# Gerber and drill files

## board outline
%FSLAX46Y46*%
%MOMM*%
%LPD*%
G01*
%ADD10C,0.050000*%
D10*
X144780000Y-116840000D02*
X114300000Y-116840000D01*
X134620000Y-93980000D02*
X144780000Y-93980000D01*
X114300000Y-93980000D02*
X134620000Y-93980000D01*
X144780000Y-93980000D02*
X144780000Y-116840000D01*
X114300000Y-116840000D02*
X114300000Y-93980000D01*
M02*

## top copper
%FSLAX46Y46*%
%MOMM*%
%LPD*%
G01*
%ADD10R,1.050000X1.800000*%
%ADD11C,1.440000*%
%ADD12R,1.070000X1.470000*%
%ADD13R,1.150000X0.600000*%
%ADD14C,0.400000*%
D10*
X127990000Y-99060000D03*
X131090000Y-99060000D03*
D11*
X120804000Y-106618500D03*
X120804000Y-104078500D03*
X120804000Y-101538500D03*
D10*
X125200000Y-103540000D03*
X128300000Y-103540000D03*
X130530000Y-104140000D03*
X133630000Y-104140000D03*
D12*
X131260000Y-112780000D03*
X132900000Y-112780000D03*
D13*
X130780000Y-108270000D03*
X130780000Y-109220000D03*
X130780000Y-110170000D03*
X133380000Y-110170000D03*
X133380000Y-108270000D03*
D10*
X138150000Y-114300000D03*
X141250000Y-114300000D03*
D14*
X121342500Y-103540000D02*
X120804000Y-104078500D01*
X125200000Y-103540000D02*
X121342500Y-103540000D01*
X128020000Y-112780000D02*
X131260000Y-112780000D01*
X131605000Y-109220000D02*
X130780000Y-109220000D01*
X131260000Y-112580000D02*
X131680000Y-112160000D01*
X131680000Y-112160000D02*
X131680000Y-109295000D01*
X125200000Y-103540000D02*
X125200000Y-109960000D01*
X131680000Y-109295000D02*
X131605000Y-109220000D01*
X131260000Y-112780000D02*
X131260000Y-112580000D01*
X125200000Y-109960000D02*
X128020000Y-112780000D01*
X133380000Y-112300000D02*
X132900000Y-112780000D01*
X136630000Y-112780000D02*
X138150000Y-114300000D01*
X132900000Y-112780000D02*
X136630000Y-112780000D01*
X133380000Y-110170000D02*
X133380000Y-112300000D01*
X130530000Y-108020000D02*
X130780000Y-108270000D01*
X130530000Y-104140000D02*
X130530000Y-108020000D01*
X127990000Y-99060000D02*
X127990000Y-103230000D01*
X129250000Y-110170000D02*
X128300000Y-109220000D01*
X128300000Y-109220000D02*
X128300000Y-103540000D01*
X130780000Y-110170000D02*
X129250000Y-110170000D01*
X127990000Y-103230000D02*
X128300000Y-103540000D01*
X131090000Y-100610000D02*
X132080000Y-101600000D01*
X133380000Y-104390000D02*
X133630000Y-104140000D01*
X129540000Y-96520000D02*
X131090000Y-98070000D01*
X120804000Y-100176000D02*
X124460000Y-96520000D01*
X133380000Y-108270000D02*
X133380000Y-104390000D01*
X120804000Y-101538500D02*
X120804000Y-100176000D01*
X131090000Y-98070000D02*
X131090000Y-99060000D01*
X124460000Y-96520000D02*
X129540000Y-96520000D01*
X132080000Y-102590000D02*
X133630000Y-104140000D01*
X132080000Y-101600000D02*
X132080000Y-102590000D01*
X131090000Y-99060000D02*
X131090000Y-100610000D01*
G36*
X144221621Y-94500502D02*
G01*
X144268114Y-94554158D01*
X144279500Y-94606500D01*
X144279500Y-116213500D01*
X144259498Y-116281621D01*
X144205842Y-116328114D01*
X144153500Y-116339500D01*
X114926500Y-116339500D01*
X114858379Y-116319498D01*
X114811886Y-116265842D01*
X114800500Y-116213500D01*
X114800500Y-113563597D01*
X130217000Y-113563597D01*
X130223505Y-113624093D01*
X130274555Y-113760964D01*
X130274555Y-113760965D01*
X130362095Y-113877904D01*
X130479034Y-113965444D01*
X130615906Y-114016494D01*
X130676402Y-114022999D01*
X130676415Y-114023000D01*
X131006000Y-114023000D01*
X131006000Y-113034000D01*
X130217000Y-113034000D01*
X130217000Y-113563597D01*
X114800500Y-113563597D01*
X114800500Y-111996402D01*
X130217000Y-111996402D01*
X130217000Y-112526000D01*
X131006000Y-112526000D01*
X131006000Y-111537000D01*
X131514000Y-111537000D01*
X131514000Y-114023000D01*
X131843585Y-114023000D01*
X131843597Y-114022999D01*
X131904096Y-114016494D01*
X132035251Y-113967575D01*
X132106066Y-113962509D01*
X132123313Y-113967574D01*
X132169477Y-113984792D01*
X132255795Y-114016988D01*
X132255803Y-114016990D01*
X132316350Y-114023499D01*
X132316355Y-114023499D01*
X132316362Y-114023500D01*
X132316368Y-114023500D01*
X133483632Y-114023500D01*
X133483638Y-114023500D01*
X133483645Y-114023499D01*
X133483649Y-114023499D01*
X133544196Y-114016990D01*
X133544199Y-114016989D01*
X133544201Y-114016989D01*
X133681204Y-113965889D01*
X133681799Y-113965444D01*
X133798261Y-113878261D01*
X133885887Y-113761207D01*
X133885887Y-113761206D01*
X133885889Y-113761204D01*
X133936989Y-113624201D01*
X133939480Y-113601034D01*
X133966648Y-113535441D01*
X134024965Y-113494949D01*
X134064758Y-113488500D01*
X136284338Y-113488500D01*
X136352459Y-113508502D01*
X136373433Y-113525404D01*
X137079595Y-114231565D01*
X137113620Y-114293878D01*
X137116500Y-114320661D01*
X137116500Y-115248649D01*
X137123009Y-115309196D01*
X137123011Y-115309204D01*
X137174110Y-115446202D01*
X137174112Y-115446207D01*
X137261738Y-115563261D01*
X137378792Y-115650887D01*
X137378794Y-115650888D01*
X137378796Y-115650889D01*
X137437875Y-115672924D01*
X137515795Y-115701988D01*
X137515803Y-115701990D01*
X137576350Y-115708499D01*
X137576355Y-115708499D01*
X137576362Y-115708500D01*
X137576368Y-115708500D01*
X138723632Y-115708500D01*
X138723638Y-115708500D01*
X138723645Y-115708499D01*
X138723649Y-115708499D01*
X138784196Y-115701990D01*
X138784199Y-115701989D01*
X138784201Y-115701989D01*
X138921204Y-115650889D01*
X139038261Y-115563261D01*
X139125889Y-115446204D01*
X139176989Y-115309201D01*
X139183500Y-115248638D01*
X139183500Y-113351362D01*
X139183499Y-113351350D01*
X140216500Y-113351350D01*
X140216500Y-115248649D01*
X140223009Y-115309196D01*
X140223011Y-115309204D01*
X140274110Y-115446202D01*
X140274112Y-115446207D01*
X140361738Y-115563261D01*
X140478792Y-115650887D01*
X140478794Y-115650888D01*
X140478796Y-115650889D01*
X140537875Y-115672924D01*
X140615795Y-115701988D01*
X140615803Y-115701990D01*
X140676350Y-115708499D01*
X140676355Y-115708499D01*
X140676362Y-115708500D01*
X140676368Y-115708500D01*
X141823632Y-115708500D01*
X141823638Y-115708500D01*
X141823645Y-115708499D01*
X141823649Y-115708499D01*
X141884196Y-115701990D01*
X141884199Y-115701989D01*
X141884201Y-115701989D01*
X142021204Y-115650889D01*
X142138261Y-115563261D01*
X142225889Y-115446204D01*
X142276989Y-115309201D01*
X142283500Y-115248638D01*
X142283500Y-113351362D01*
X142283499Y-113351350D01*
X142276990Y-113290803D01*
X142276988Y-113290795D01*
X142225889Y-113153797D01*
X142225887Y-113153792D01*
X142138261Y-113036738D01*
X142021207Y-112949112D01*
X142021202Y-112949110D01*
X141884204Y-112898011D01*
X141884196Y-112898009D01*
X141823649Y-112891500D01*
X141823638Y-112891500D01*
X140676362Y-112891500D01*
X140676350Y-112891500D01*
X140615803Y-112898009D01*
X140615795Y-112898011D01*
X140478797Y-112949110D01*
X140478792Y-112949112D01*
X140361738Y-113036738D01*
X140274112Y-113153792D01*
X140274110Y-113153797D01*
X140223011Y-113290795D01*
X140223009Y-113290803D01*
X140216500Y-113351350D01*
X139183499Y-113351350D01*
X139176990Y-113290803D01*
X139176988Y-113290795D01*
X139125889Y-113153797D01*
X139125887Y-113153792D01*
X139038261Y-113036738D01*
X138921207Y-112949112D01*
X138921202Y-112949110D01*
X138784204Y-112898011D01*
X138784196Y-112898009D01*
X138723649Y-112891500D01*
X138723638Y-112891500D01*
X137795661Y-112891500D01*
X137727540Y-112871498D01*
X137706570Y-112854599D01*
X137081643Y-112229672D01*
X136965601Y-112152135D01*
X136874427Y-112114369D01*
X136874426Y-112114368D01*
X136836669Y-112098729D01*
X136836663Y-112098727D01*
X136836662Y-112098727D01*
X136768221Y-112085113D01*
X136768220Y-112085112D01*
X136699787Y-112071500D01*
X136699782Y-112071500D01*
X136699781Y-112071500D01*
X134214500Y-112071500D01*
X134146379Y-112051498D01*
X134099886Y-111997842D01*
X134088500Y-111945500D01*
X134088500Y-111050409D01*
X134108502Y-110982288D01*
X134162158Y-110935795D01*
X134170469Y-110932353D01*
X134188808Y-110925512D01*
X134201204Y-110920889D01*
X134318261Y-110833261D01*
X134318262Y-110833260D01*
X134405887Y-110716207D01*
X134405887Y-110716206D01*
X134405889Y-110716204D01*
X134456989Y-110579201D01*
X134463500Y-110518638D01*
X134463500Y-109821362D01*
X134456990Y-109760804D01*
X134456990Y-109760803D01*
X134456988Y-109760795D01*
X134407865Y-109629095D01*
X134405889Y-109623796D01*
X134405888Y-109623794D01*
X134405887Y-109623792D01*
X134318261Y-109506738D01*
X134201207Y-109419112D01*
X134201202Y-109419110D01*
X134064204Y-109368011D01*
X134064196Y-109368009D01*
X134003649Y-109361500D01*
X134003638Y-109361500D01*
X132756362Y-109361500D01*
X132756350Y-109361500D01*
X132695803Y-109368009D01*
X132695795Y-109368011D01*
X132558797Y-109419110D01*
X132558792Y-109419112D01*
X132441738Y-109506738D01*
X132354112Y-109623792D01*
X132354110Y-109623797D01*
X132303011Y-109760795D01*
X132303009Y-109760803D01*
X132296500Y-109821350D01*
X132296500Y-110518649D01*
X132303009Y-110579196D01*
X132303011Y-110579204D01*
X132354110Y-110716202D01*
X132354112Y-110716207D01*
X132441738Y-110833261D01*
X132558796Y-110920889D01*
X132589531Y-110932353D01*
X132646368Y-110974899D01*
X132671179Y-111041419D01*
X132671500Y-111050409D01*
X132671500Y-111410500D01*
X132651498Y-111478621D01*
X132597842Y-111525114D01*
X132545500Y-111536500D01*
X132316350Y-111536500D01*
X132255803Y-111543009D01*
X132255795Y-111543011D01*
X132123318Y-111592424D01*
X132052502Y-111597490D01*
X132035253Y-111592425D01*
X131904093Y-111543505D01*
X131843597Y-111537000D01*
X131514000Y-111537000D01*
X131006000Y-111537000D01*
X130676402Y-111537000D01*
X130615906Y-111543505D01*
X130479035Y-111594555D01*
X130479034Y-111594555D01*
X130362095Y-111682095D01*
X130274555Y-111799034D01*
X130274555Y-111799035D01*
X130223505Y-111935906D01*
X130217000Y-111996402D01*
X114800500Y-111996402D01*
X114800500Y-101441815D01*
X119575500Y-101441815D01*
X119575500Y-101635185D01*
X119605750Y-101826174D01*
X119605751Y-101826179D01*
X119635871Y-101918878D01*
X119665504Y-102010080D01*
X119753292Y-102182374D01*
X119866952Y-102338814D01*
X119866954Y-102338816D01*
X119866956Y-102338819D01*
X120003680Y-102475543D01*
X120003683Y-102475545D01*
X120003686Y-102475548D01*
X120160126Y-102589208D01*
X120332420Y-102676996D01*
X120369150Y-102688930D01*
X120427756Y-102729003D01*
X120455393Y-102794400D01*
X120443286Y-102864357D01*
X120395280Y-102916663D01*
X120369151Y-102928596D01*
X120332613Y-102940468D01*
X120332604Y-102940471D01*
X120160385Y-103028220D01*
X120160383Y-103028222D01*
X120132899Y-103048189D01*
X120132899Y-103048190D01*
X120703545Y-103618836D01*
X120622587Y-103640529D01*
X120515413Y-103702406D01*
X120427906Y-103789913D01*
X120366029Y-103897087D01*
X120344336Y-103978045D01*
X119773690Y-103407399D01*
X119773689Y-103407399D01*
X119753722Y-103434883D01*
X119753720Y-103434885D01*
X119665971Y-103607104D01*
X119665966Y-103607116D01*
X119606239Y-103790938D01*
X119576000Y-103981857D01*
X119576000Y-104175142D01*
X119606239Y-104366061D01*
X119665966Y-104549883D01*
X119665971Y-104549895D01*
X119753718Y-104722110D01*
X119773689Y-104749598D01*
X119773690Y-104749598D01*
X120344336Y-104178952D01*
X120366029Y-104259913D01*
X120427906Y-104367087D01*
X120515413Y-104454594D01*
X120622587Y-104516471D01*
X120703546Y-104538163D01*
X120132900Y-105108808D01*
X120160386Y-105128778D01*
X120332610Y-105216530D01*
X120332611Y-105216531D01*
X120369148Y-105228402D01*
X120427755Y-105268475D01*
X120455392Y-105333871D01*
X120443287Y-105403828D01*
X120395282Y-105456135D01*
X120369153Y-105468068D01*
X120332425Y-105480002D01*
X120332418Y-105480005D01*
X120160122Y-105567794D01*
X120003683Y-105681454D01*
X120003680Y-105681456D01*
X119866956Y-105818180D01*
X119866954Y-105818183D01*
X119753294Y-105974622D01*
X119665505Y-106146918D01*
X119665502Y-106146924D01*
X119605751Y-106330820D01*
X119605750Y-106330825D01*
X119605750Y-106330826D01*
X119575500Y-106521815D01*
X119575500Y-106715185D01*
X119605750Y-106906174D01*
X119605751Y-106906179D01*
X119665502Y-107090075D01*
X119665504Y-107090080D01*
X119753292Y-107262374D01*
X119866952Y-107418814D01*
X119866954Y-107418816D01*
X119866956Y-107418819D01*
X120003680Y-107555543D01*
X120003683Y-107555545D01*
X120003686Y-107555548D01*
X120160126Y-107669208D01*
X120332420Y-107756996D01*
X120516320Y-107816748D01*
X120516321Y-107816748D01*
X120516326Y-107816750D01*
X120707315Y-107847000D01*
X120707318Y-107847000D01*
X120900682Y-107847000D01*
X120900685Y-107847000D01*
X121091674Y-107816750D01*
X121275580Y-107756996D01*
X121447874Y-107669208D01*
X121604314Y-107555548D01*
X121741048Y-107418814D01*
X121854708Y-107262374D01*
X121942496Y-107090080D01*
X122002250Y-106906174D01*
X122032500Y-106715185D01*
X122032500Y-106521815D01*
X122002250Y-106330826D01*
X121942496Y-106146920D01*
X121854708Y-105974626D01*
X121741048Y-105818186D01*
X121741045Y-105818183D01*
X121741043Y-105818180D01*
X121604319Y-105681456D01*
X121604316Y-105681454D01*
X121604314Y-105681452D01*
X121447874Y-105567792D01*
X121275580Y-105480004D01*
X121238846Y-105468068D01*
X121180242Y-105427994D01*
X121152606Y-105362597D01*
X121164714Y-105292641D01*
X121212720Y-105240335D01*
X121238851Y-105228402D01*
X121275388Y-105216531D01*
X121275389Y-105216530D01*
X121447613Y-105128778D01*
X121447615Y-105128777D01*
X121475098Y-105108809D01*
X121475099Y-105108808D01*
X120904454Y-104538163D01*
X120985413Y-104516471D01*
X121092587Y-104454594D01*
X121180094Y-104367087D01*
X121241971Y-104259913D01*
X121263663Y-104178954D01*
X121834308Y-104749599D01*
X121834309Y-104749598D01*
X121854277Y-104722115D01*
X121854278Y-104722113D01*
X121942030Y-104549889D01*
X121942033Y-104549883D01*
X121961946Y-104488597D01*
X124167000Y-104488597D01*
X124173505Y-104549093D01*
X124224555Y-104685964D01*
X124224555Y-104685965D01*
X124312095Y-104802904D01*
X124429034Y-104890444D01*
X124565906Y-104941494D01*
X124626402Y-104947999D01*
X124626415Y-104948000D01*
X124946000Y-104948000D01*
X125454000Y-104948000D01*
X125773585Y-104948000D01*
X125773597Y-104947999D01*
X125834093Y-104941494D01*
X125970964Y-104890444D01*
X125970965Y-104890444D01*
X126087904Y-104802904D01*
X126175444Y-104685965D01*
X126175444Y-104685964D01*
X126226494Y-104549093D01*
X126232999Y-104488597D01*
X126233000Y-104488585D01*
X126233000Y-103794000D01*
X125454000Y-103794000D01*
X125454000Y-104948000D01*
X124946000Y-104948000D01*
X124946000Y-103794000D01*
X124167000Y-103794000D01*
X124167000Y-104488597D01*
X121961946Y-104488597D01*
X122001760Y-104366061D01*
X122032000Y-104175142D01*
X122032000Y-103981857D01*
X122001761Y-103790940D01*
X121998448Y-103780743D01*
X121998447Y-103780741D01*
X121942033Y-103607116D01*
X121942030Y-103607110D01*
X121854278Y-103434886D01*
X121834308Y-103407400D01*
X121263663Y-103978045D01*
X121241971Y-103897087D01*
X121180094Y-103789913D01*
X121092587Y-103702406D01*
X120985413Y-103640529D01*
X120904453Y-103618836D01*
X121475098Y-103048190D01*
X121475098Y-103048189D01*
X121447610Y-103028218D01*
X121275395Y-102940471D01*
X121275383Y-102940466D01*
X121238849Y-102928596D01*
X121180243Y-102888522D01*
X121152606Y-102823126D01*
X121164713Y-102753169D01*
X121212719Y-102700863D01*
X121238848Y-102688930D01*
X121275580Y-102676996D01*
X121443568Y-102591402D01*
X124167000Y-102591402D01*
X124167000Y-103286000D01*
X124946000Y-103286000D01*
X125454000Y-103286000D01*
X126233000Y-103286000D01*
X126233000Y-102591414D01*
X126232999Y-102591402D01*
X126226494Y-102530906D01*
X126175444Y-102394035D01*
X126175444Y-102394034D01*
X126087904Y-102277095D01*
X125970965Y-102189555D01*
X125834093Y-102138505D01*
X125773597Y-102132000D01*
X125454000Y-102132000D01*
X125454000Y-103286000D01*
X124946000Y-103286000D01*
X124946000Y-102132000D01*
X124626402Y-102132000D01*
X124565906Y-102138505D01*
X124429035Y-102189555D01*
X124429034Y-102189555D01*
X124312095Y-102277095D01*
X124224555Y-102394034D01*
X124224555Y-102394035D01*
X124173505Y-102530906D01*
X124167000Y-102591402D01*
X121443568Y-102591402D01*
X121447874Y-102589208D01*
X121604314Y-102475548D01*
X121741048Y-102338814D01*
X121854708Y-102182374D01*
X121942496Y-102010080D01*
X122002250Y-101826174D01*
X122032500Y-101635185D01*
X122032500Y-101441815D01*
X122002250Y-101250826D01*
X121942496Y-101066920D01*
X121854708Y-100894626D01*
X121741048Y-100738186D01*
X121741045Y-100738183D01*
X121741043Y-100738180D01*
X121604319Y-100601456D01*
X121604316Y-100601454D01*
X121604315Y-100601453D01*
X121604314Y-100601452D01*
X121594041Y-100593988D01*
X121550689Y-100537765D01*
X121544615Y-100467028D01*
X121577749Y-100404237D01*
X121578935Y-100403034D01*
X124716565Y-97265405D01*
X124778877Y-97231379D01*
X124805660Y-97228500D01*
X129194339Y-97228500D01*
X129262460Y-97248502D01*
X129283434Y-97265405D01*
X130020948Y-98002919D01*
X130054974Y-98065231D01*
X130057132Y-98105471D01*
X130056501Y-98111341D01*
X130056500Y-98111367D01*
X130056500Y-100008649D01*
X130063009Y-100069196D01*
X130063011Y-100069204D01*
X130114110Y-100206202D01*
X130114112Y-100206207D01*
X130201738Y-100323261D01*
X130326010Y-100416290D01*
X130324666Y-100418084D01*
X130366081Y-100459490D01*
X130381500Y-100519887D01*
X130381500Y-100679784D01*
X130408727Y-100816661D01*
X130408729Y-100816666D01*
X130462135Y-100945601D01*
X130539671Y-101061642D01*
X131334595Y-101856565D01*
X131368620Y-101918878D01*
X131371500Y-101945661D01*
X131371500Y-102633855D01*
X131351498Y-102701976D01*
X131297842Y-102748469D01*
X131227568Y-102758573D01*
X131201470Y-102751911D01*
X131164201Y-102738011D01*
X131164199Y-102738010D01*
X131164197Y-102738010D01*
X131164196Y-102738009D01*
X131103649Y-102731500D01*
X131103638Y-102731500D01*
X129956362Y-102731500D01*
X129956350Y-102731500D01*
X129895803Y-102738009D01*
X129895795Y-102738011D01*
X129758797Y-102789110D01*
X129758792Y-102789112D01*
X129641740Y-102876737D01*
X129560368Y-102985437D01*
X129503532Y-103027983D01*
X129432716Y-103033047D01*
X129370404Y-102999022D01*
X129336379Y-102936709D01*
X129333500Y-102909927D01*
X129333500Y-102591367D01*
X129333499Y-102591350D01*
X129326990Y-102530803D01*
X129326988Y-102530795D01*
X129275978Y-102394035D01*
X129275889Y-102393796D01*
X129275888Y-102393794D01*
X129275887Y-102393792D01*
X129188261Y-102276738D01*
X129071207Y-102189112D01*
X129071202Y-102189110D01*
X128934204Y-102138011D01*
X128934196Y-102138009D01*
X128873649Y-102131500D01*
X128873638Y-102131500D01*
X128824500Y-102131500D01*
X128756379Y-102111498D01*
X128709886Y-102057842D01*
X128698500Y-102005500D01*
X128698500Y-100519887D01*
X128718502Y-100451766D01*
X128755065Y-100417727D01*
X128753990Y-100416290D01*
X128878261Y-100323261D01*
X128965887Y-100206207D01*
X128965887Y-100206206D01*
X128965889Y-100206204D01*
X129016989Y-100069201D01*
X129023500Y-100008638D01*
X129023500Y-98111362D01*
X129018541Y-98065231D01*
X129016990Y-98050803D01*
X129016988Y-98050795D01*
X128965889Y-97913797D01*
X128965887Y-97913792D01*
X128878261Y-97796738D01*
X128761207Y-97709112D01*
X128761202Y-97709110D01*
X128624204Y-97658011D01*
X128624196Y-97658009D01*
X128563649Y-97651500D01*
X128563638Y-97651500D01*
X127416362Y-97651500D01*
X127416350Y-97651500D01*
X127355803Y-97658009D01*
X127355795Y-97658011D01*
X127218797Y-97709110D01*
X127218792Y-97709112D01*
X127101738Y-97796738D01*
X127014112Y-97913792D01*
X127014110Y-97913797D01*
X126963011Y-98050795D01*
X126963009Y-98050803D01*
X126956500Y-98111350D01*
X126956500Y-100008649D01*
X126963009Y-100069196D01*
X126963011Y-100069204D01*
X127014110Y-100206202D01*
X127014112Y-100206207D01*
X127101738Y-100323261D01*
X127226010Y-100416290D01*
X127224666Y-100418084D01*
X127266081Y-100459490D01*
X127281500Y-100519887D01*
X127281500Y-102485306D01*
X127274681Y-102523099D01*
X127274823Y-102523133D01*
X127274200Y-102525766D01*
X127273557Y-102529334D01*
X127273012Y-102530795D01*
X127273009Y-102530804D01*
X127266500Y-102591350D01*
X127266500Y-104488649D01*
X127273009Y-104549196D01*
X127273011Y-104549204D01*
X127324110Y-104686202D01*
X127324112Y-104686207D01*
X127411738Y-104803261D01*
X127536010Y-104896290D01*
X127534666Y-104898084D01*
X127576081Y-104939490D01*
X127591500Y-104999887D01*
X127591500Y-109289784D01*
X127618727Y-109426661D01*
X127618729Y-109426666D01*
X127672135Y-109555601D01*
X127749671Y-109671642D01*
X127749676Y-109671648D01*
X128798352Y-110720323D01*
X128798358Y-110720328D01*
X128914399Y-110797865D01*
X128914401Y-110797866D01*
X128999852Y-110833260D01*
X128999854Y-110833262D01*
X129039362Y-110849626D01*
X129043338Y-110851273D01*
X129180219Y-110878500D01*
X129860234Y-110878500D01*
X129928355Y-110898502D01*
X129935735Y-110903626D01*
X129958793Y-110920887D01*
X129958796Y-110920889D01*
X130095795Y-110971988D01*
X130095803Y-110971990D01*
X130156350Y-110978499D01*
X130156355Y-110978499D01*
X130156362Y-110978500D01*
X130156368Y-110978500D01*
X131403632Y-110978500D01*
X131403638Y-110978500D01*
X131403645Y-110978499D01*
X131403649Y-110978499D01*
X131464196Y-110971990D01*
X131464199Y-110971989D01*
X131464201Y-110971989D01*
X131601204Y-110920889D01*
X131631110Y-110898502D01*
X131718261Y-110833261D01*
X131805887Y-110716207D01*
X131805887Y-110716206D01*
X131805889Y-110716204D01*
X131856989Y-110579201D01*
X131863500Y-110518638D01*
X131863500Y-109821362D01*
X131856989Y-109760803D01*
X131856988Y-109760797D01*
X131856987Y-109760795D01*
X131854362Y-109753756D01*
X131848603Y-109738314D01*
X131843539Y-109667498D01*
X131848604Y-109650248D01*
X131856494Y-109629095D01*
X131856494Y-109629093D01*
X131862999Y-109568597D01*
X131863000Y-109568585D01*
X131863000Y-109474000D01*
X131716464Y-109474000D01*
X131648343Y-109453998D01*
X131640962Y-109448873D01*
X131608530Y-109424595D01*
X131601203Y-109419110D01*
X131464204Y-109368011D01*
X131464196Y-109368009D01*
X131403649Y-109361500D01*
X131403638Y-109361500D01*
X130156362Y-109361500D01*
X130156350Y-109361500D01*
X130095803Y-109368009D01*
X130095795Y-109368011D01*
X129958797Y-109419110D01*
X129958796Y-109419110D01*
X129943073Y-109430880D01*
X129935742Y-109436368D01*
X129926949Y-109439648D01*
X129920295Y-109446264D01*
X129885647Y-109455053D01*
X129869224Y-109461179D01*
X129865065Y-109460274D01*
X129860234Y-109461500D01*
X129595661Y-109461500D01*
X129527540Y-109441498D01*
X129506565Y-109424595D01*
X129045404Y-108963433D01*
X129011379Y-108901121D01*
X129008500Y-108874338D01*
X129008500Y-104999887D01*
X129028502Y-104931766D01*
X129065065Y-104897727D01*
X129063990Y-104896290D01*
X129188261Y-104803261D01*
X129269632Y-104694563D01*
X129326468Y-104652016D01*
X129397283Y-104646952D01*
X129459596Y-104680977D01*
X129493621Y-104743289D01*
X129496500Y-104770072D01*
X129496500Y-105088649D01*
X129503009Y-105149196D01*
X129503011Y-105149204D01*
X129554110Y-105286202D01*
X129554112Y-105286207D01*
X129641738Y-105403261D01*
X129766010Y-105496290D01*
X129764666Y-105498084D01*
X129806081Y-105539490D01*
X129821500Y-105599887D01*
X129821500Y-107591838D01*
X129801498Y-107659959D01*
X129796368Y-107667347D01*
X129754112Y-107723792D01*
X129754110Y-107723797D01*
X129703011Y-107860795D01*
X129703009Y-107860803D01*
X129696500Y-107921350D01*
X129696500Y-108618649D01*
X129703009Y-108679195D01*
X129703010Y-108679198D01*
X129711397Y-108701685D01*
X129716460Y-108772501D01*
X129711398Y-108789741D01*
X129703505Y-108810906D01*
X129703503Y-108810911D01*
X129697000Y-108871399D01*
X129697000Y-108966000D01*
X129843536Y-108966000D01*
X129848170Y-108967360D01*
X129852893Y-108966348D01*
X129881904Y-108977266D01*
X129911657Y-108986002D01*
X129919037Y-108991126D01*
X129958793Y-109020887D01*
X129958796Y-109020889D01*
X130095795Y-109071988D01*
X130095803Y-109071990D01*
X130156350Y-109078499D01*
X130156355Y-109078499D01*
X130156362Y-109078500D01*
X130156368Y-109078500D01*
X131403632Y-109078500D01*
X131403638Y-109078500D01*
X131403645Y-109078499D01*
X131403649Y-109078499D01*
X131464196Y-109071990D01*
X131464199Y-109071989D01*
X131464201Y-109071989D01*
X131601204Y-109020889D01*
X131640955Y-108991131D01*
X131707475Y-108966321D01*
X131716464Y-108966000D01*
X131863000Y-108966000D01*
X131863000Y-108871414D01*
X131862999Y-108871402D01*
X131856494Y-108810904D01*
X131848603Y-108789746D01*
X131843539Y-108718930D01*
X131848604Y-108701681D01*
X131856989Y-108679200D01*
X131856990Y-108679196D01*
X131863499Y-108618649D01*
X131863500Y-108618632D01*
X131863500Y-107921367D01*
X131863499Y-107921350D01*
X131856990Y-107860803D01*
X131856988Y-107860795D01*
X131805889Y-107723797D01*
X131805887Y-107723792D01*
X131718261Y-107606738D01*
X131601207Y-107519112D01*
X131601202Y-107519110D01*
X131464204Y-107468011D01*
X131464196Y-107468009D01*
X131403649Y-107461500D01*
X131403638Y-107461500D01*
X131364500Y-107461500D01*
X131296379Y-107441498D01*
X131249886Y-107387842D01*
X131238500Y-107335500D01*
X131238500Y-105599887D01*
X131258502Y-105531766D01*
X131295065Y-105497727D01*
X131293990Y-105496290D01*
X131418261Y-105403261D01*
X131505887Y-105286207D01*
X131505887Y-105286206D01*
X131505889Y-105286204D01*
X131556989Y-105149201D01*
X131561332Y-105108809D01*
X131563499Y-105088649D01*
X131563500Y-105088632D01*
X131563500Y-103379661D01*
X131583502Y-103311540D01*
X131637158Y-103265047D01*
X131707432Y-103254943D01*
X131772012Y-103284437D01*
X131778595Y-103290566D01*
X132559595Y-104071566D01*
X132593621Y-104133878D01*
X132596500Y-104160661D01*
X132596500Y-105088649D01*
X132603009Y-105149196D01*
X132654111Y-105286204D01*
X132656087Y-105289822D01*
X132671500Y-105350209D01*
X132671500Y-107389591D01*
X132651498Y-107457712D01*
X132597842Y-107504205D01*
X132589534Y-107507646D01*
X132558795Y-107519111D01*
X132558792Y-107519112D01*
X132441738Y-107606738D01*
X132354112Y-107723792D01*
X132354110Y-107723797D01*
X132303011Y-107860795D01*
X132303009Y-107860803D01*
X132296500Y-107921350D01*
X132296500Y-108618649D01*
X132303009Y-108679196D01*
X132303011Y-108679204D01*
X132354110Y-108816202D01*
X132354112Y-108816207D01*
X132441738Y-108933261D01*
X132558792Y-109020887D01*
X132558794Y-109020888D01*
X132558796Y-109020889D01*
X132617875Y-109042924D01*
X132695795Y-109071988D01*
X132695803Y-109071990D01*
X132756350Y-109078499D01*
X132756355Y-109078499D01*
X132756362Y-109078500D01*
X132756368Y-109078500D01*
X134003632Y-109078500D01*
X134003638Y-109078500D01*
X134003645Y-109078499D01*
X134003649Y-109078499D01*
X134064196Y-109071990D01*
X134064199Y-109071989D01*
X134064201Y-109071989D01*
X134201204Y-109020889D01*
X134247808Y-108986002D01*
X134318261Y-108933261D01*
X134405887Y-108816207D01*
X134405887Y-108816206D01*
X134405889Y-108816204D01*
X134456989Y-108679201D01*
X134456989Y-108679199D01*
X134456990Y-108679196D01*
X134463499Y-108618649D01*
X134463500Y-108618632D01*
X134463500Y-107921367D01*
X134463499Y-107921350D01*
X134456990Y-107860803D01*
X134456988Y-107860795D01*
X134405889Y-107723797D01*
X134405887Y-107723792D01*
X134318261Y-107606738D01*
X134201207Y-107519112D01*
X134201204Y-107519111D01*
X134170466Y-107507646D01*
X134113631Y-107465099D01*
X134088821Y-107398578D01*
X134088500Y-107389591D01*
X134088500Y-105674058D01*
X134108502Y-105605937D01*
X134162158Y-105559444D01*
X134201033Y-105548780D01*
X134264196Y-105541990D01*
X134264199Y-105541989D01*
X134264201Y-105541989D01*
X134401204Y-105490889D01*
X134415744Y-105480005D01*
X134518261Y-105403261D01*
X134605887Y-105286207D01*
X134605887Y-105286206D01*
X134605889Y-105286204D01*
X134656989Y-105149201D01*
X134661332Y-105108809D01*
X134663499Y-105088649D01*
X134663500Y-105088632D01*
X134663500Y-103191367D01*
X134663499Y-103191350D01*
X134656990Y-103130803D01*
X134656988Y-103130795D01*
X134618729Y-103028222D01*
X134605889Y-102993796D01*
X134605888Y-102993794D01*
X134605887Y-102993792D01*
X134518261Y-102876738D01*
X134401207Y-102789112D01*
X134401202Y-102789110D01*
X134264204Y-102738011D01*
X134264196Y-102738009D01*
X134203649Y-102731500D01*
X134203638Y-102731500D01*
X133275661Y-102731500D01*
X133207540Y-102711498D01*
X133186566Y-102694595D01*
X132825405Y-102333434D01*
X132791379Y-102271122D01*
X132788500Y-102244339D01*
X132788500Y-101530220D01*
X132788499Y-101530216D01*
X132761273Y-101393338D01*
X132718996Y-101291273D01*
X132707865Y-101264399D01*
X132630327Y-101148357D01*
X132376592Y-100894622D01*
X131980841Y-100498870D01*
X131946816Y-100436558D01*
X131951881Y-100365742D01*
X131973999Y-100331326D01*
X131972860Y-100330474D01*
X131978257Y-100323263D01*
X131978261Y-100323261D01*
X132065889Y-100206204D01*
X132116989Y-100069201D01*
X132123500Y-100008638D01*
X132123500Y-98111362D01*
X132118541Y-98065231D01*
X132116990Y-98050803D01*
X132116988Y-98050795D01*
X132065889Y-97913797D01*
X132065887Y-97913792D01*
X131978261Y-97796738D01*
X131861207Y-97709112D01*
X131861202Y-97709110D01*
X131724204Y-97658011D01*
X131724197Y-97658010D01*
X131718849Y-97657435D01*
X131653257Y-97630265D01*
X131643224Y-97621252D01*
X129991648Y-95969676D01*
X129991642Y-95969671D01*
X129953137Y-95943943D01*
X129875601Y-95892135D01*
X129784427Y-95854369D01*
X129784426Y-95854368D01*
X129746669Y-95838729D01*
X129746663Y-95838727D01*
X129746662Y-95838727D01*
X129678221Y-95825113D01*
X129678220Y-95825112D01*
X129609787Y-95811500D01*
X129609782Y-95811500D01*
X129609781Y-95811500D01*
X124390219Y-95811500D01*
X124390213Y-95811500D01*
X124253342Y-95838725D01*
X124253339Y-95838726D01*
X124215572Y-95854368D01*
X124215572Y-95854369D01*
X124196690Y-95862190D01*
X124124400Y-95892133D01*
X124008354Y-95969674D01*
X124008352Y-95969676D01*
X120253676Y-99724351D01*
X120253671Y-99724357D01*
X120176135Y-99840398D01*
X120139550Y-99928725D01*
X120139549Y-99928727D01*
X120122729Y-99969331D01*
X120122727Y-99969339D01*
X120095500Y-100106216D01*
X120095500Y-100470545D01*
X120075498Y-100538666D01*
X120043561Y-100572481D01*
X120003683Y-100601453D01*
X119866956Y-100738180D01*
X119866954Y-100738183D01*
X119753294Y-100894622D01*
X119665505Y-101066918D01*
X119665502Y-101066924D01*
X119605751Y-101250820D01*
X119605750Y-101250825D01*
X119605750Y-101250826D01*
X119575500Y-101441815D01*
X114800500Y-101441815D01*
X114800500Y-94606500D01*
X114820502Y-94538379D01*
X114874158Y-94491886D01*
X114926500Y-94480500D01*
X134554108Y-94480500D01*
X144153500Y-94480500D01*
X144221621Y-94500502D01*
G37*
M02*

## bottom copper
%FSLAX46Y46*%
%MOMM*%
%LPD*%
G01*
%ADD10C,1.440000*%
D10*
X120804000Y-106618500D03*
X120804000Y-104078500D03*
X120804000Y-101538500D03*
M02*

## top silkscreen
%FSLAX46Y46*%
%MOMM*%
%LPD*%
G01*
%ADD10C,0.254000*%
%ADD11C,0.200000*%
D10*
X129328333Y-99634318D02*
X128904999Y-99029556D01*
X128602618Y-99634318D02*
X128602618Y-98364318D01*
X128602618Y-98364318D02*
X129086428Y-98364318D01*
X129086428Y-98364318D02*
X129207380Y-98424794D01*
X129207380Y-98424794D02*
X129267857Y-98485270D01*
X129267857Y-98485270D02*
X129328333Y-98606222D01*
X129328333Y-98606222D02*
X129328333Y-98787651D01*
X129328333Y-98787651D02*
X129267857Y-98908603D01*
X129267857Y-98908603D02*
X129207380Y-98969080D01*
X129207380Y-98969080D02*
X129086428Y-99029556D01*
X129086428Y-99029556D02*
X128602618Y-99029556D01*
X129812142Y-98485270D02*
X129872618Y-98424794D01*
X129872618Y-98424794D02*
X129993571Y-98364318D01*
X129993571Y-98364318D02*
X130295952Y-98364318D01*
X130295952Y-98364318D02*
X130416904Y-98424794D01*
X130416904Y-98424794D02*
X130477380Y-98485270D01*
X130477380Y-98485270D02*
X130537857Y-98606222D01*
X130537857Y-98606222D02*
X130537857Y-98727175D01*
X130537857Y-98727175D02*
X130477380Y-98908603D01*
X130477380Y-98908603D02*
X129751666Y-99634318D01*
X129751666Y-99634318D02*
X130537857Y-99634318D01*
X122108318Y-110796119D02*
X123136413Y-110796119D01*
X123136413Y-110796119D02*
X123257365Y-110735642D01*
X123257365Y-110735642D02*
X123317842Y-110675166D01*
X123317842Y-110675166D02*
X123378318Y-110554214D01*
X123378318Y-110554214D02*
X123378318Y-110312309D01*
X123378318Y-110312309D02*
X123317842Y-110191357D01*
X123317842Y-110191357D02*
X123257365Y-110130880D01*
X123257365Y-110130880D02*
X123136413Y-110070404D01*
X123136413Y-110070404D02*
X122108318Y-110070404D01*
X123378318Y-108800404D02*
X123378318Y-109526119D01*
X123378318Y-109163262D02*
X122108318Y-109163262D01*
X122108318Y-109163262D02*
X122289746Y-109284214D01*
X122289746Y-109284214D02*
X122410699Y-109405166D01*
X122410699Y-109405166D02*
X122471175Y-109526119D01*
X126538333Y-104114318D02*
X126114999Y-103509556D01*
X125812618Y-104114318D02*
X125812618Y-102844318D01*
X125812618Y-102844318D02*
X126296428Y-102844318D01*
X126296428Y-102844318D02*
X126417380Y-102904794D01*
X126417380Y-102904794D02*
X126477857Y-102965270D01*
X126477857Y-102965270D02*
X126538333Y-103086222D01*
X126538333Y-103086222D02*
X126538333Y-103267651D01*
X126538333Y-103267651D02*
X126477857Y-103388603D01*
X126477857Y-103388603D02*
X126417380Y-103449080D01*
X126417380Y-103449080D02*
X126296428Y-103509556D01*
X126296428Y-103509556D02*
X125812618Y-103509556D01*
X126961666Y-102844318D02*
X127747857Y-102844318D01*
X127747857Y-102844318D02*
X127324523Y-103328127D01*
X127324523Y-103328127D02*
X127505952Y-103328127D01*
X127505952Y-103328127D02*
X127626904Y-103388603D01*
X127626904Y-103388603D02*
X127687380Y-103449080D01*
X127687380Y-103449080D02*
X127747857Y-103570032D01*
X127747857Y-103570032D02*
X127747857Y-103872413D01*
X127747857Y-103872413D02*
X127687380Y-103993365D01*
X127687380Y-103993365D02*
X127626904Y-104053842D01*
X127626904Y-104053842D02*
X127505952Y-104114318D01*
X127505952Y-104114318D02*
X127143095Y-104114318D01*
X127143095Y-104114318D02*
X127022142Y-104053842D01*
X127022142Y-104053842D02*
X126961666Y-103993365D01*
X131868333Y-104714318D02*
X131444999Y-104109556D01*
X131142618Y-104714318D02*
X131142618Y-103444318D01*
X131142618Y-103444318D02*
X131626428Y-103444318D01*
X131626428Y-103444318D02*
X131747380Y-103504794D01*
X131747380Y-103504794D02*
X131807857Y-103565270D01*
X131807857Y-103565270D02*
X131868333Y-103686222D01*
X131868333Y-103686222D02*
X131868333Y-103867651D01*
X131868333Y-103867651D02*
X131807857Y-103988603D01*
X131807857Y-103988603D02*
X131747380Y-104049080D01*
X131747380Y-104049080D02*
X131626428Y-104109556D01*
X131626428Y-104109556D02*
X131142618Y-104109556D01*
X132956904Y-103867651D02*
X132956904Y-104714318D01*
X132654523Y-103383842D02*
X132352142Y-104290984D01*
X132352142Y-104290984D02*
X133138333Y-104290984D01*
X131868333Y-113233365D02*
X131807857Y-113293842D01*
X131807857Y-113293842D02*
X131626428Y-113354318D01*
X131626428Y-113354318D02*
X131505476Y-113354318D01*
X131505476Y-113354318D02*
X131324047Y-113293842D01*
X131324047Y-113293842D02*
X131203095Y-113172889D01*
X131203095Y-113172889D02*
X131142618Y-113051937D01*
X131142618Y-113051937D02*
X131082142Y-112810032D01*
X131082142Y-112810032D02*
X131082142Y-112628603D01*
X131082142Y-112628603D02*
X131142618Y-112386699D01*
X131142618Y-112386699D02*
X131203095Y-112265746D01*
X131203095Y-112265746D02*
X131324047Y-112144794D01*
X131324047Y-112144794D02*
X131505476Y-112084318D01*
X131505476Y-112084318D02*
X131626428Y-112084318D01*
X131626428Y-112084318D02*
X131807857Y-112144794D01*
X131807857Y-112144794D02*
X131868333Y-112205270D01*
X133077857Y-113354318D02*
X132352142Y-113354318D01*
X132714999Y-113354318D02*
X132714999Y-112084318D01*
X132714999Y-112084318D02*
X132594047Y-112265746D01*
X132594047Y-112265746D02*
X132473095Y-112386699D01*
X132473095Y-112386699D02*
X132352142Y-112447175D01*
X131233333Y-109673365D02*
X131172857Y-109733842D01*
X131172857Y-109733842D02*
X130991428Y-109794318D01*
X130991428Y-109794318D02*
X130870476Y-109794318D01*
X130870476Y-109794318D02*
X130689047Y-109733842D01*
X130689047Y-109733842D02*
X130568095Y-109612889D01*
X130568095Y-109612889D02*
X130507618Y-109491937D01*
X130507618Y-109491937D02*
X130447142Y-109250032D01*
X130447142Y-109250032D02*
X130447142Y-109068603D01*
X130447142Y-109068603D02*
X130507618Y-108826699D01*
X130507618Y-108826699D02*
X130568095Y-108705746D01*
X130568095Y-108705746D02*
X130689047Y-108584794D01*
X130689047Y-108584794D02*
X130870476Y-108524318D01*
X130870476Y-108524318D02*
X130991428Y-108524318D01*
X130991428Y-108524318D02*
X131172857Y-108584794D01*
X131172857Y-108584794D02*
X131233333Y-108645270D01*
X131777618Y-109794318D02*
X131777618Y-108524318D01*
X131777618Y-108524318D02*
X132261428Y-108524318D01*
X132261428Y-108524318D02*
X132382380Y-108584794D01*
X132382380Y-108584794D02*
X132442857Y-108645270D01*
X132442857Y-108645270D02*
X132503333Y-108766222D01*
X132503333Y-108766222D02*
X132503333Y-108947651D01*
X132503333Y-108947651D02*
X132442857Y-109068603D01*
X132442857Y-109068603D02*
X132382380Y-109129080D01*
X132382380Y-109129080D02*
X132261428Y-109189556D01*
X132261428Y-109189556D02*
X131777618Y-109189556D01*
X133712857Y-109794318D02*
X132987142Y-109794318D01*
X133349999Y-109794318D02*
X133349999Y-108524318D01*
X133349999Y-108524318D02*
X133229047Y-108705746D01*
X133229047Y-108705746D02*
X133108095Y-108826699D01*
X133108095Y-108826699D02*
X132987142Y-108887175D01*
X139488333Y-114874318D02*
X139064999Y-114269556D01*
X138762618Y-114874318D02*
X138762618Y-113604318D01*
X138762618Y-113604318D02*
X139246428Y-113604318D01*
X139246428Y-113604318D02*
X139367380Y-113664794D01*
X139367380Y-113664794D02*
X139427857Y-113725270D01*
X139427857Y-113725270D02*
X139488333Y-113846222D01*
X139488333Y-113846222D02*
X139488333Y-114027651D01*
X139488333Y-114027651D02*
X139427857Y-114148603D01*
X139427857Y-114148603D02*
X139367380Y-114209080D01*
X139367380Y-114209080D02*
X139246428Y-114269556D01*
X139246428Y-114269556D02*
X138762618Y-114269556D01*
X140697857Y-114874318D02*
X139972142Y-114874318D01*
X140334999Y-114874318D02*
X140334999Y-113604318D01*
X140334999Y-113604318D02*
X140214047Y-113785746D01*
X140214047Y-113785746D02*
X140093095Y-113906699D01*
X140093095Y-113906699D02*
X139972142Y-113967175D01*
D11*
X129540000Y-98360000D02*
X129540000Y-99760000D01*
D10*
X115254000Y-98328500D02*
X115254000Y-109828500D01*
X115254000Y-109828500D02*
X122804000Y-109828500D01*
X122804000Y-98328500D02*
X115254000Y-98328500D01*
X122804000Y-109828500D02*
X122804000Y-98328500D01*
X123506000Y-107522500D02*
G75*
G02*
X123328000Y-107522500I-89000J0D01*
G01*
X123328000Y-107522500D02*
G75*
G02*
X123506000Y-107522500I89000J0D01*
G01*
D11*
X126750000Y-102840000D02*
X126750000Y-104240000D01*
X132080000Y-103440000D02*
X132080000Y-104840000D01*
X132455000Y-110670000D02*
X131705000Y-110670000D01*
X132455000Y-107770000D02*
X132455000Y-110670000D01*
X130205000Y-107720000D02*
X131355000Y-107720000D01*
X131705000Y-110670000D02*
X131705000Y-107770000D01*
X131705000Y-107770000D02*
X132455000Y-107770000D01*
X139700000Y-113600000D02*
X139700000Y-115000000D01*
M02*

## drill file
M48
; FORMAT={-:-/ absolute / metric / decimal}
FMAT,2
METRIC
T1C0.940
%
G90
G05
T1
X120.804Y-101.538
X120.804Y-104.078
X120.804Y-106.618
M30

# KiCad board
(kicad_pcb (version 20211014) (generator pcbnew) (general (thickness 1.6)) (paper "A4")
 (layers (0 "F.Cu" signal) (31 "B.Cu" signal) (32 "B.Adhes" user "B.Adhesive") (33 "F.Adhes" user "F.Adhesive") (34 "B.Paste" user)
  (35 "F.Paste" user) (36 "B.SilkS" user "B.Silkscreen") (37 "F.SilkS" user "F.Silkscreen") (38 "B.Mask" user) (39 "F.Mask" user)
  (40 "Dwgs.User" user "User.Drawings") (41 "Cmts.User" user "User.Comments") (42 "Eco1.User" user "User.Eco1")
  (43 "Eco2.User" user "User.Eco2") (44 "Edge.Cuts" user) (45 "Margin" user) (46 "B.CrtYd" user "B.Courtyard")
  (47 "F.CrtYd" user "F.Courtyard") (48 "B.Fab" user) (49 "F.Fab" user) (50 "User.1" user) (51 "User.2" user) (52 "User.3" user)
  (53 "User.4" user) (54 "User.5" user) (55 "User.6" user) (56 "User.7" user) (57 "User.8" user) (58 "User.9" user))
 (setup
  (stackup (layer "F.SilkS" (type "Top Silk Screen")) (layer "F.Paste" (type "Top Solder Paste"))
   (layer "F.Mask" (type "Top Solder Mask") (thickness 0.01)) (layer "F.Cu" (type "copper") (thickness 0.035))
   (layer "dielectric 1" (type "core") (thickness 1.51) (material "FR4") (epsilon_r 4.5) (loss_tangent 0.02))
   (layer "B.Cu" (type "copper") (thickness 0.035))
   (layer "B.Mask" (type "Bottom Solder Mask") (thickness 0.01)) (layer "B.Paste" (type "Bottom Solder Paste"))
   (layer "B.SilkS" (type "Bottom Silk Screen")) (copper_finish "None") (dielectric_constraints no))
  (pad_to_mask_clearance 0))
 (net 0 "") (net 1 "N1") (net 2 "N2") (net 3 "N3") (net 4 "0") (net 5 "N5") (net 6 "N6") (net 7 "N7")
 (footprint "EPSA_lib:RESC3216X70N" (layer "F.Cu") (at 129.54 99.06)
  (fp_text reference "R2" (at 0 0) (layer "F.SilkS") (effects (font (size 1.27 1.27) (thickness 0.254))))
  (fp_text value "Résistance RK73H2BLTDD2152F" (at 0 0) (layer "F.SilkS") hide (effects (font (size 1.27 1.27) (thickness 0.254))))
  (fp_line (start 0 -0.7) (end 0 0.7) (layer "F.SilkS") (width 0.2))
  (pad "1" smd rect (at -1.55 0) (size 1.05 1.8) (layers "F.Cu" "F.Paste" "F.Mask") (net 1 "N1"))
  (pad "2" smd rect (at 1.55 0) (size 1.05 1.8) (layers "F.Cu" "F.Paste" "F.Mask") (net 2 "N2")))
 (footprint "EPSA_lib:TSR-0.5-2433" (layer "F.Cu") (at 122.804 109.8285 90)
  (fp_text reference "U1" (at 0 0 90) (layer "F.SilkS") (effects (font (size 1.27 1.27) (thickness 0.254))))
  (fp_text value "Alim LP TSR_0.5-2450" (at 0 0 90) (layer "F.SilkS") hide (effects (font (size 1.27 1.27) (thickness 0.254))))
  (fp_line (start 11.5 -7.55) (end 0 -7.55) (layer "F.SilkS") (width 0.254))
  (fp_line (start 0 -7.55) (end 0 0) (layer "F.SilkS") (width 0.254))
  (fp_line (start 11.5 0) (end 11.5 -7.55) (layer "F.SilkS") (width 0.254))
  (fp_line (start 0 0) (end 11.5 0) (layer "F.SilkS") (width 0.254))
  (fp_circle (center 2.306 0.613) (end 2.306 0.702) (layer "F.SilkS") (width 0.254) (fill none))
  (pad "1" thru_hole circle (at 3.21 -2 90) (size 1.44 1.44) (drill 0.94) (layers *.Cu *.Mask) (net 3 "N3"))
  (pad "2" thru_hole circle (at 5.75 -2 90) (size 1.44 1.44) (drill 0.94) (layers *.Cu *.Mask) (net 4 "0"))
  (pad "3" thru_hole circle (at 8.29 -2 90) (size 1.44 1.44) (drill 0.94) (layers *.Cu *.Mask) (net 2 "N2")))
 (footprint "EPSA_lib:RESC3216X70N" (layer "F.Cu") (at 126.75 103.54)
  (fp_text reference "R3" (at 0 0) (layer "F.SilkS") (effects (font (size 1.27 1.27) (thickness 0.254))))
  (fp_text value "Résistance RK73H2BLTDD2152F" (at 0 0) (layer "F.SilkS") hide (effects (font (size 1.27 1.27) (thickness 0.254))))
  (fp_line (start 0 -0.7) (end 0 0.7) (layer "F.SilkS") (width 0.2))
  (pad "1" smd rect (at -1.55 0) (size 1.05 1.8) (layers "F.Cu" "F.Paste" "F.Mask") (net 4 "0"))
  (pad "2" smd rect (at 1.55 0) (size 1.05 1.8) (layers "F.Cu" "F.Paste" "F.Mask") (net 1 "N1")))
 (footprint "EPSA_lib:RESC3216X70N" (layer "F.Cu") (at 132.08 104.14)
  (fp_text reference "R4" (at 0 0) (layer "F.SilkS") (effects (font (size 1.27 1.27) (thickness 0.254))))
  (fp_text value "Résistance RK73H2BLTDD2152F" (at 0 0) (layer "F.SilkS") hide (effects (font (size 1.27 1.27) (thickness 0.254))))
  (fp_line (start 0 -0.7) (end 0 0.7) (layer "F.SilkS") (width 0.2))
  (pad "1" smd rect (at -1.55 0) (size 1.05 1.8) (layers "F.Cu" "F.Paste" "F.Mask") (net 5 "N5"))
  (pad "2" smd rect (at 1.55 0) (size 1.05 1.8) (layers "F.Cu" "F.Paste" "F.Mask") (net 2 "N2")))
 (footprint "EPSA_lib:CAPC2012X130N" (layer "F.Cu") (at 132.08 112.78)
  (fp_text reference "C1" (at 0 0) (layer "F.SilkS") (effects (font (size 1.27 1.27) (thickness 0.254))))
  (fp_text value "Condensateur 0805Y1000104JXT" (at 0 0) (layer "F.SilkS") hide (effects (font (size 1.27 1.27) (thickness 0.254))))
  (pad "1" smd rect (at -0.82 0) (size 1.07 1.47) (layers "F.Cu" "F.Paste" "F.Mask") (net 4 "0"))
  (pad "2" smd rect (at 0.82 0) (size 1.07 1.47) (layers "F.Cu" "F.Paste" "F.Mask") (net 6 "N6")))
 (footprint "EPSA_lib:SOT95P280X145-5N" (layer "F.Cu") (at 132.08 109.22)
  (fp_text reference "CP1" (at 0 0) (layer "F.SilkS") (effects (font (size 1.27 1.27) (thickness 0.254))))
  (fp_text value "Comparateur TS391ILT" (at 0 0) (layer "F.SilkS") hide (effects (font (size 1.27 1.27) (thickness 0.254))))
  (fp_line (start 0.375 1.45) (end -0.375 1.45) (layer "F.SilkS") (width 0.2))
  (fp_line (start 0.375 -1.45) (end 0.375 1.45) (layer "F.SilkS") (width 0.2))
  (fp_line (start -1.875 -1.5) (end -0.725 -1.5) (layer "F.SilkS") (width 0.2))
  (fp_line (start -0.375 1.45) (end -0.375 -1.45) (layer "F.SilkS") (width 0.2))
  (fp_line (start -0.375 -1.45) (end 0.375 -1.45) (layer "F.SilkS") (width 0.2))
  (pad "1" smd rect (at -1.3 -0.95 90) (size 0.6 1.15) (layers "F.Cu" "F.Paste" "F.Mask") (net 5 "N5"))
  (pad "2" smd rect (at -1.3 0 90) (size 0.6 1.15) (layers "F.Cu" "F.Paste" "F.Mask") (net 4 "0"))
  (pad "3" smd rect (at -1.3 0.95 90) (size 0.6 1.15) (layers "F.Cu" "F.Paste" "F.Mask") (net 1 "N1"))
  (pad "4" smd rect (at 1.3 0.95 90) (size 0.6 1.15) (layers "F.Cu" "F.Paste" "F.Mask") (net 6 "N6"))
  (pad "5" smd rect (at 1.3 -0.95 90) (size 0.6 1.15) (layers "F.Cu" "F.Paste" "F.Mask") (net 2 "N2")))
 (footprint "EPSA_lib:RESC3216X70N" (layer "F.Cu") (at 139.7 114.3)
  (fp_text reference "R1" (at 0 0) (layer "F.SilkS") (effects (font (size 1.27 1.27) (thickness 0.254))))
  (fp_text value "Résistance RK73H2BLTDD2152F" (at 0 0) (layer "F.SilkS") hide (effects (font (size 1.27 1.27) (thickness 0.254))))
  (fp_line (start 0 -0.7) (end 0 0.7) (layer "F.SilkS") (width 0.2))
  (pad "1" smd rect (at -1.55 0) (size 1.05 1.8) (layers "F.Cu" "F.Paste" "F.Mask") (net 6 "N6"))
  (pad "2" smd rect (at 1.55 0) (size 1.05 1.8) (layers "F.Cu" "F.Paste" "F.Mask") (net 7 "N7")))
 (gr_line (start 144.78 116.84) (end 114.3 116.84) (layer "Edge.Cuts") (width 0.05))
 (gr_line (start 134.62 93.98) (end 144.78 93.98) (layer "Edge.Cuts") (width 0.05))
 (gr_line (start 114.3 93.98) (end 134.62 93.98) (layer "Edge.Cuts") (width 0.05))
 (gr_line (start 144.78 93.98) (end 144.78 116.84) (layer "Edge.Cuts") (width 0.05))
 (gr_line (start 114.3 116.84) (end 114.3 93.98) (layer "Edge.Cuts") (width 0.05))
 (segment (start 121.3425 103.54) (end 120.804 104.0785) (width 0.4) (layer "F.Cu") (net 4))
 (segment (start 125.2 103.54) (end 121.3425 103.54) (width 0.4) (layer "F.Cu") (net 4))
 (segment (start 128.02 112.78) (end 131.26 112.78) (width 0.4) (layer "F.Cu") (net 4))
 (segment (start 131.605 109.22) (end 130.78 109.22) (width 0.4) (layer "F.Cu") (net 4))
 (segment (start 131.26 112.58) (end 131.68 112.16) (width 0.4) (layer "F.Cu") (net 4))
 (segment (start 131.68 112.16) (end 131.68 109.295) (width 0.4) (layer "F.Cu") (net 4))
 (segment (start 125.2 103.54) (end 125.2 109.96) (width 0.4) (layer "F.Cu") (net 4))
 (segment (start 131.68 109.295) (end 131.605 109.22) (width 0.4) (layer "F.Cu") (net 4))
 (segment (start 131.26 112.78) (end 131.26 112.58) (width 0.4) (layer "F.Cu") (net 4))
 (segment (start 125.2 109.96) (end 128.02 112.78) (width 0.4) (layer "F.Cu") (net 4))
 (segment (start 133.38 112.3) (end 132.9 112.78) (width 0.4) (layer "F.Cu") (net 6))
 (segment (start 136.63 112.78) (end 138.15 114.3) (width 0.4) (layer "F.Cu") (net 6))
 (segment (start 132.9 112.78) (end 136.63 112.78) (width 0.4) (layer "F.Cu") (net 6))
 (segment (start 133.38 110.17) (end 133.38 112.3) (width 0.4) (layer "F.Cu") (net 6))
 (segment (start 130.53 108.02) (end 130.78 108.27) (width 0.4) (layer "F.Cu") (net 5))
 (segment (start 130.53 104.14) (end 130.53 108.02) (width 0.4) (layer "F.Cu") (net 5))
 (segment (start 127.99 99.06) (end 127.99 103.23) (width 0.4) (layer "F.Cu") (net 1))
 (segment (start 129.25 110.17) (end 128.3 109.22) (width 0.4) (layer "F.Cu") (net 1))
 (segment (start 128.3 109.22) (end 128.3 103.54) (width 0.4) (layer "F.Cu") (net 1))
 (segment (start 130.78 110.17) (end 129.25 110.17) (width 0.4) (layer "F.Cu") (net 1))
 (segment (start 127.99 103.23) (end 128.3 103.54) (width 0.4) (layer "F.Cu") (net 1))
 (segment (start 131.09 100.61) (end 132.08 101.6) (width 0.4) (layer "F.Cu") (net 2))
 (segment (start 133.38 104.39) (end 133.63 104.14) (width 0.4) (layer "F.Cu") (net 2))
 (segment (start 129.54 96.52) (end 131.09 98.07) (width 0.4) (layer "F.Cu") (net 2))
 (segment (start 120.804 100.176) (end 124.46 96.52) (width 0.4) (layer "F.Cu") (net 2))
 (segment (start 133.38 108.27) (end 133.38 104.39) (width 0.4) (layer "F.Cu") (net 2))
 (segment (start 120.804 101.5385) (end 120.804 100.176) (width 0.4) (layer "F.Cu") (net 2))
 (segment (start 131.09 98.07) (end 131.09 99.06) (width 0.4) (layer "F.Cu") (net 2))
 (segment (start 124.46 96.52) (end 129.54 96.52) (width 0.4) (layer "F.Cu") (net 2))
 (segment (start 132.08 102.59) (end 133.63 104.14) (width 0.4) (layer "F.Cu") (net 2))
 (segment (start 132.08 101.6) (end 132.08 102.59) (width 0.4) (layer "F.Cu") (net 2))
 (segment (start 131.09 99.06) (end 131.09 100.61) (width 0.4) (layer "F.Cu") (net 2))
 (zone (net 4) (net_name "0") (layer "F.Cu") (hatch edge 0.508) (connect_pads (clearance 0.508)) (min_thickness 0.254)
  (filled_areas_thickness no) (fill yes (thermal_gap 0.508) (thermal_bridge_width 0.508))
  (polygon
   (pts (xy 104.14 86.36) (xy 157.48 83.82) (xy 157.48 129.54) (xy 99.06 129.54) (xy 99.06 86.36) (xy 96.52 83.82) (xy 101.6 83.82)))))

